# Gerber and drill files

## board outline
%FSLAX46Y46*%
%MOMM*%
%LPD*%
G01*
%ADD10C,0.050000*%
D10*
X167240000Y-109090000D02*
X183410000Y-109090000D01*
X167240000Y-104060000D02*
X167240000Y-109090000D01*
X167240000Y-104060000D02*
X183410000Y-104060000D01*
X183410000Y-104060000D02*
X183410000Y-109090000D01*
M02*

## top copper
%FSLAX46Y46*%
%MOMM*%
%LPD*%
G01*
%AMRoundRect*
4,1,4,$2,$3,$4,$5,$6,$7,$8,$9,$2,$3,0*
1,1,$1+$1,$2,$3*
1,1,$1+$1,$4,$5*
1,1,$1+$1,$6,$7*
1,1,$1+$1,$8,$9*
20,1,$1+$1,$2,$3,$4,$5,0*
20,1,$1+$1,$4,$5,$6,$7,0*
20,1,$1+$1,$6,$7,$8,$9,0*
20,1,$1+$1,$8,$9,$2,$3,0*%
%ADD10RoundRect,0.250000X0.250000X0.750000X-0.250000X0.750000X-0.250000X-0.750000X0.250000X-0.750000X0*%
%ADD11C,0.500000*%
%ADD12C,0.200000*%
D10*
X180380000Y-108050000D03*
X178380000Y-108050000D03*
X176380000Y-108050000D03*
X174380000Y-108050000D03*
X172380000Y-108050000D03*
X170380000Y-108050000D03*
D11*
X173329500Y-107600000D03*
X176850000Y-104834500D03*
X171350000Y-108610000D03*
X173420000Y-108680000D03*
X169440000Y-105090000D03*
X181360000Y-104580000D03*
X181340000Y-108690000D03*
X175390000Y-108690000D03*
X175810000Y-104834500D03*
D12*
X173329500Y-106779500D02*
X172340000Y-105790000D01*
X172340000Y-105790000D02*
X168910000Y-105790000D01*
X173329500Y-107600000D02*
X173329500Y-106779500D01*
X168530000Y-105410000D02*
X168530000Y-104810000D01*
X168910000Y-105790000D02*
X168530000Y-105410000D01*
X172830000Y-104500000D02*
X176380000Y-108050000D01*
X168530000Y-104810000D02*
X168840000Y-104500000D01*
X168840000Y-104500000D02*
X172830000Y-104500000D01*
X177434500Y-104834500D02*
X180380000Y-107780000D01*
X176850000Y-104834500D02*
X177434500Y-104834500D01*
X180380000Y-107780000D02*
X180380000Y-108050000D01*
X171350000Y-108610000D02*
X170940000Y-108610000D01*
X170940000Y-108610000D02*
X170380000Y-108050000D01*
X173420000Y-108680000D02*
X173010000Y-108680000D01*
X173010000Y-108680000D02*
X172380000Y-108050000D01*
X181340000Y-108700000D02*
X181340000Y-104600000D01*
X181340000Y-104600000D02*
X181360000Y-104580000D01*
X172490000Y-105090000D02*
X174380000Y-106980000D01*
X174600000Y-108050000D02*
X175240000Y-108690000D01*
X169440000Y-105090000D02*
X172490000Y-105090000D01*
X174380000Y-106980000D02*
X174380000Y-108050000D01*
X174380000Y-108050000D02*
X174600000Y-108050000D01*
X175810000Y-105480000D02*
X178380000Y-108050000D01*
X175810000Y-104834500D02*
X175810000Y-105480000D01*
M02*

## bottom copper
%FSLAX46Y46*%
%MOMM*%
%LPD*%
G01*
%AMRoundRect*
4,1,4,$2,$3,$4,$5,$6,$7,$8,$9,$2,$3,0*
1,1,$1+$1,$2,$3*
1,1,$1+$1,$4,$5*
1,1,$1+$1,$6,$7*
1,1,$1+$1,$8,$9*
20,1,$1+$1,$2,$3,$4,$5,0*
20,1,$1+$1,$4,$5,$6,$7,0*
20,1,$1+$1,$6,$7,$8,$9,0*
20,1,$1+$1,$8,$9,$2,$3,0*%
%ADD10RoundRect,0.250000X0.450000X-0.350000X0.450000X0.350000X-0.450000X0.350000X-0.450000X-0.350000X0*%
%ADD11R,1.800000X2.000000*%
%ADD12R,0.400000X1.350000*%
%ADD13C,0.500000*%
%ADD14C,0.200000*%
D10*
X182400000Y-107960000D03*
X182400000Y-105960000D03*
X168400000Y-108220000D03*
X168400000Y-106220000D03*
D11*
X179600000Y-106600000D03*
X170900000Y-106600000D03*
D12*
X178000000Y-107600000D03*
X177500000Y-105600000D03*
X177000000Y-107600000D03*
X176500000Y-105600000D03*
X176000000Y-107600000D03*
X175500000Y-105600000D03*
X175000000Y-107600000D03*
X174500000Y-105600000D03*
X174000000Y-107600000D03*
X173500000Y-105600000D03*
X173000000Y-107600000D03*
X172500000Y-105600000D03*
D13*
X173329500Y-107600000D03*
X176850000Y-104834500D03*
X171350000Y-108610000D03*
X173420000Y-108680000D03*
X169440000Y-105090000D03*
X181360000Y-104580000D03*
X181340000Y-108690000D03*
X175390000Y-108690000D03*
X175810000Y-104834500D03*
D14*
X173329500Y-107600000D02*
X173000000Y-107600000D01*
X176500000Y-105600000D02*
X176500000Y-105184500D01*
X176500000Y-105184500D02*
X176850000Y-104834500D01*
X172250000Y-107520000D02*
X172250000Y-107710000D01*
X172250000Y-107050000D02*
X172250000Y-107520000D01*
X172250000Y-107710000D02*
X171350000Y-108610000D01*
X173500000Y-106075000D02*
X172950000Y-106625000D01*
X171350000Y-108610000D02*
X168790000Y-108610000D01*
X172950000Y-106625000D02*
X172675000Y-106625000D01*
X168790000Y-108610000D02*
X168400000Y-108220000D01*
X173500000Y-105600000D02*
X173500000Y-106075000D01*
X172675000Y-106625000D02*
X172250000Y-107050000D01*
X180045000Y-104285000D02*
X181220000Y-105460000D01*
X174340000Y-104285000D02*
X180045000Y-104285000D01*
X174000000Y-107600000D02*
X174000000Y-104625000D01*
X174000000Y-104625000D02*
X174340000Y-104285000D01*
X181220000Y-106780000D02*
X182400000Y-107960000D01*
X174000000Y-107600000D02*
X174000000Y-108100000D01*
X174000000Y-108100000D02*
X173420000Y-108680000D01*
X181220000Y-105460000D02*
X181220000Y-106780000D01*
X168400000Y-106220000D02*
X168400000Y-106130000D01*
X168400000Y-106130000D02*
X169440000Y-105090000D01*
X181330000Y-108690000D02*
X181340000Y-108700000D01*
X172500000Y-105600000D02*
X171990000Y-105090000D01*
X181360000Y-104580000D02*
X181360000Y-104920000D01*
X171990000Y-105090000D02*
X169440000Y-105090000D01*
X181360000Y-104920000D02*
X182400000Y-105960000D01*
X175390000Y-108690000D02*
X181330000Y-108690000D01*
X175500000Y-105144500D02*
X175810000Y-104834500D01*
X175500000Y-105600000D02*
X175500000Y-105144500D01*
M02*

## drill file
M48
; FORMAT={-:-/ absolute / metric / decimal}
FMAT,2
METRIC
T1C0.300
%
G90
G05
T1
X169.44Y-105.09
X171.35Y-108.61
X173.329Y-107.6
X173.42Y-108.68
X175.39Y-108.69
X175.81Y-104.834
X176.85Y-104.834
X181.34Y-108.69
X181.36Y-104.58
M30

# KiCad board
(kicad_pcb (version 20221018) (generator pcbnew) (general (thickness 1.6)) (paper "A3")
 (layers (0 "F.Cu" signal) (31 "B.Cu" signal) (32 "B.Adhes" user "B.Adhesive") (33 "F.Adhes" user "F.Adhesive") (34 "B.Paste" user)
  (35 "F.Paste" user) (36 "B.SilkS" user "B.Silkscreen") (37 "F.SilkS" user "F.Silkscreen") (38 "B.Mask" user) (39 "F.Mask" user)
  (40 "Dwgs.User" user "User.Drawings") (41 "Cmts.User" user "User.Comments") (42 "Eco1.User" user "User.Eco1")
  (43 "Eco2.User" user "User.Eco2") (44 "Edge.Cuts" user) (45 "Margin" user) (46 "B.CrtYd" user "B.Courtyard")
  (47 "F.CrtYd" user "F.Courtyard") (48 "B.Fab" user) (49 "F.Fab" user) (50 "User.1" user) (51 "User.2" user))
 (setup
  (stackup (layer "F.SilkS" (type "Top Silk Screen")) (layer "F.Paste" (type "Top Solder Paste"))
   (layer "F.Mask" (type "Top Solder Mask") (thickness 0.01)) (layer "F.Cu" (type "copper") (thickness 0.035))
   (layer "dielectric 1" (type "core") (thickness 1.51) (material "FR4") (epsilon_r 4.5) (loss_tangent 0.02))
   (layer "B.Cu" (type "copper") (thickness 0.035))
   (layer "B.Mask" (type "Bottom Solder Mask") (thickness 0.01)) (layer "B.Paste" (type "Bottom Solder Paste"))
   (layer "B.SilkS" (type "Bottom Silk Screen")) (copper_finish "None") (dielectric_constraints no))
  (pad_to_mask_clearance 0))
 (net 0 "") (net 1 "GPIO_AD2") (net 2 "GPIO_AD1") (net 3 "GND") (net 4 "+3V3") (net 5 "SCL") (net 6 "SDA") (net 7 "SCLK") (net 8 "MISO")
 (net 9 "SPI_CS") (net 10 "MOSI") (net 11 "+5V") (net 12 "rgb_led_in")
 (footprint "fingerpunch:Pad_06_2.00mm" (layer "F.Cu") (at 175.38 108.05 180)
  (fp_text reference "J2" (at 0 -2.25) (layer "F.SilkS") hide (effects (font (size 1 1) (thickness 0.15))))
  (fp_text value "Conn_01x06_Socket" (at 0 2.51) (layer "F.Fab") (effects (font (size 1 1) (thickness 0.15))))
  (pad "1" smd roundrect (at -5 0 180) (size 1 2) (layers "F.Cu" "F.Paste" "F.Mask") (roundrect_rratio 0.25) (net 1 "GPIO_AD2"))
  (pad "2" smd roundrect (at -3 0 180) (size 1 2) (layers "F.Cu" "F.Paste" "F.Mask") (roundrect_rratio 0.25) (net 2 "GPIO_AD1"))
  (pad "3" smd roundrect (at -1 0 180) (size 1 2) (layers "F.Cu" "F.Paste" "F.Mask") (roundrect_rratio 0.25) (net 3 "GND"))
  (pad "4" smd roundrect (at 1 0 180) (size 1 2) (layers "F.Cu" "F.Paste" "F.Mask") (roundrect_rratio 0.25) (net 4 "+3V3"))
  (pad "5" smd roundrect (at 3 0 180) (size 1 2) (layers "F.Cu" "F.Paste" "F.Mask") (roundrect_rratio 0.25) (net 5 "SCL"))
  (pad "6" smd roundrect (at 5 0 180) (size 1 2) (layers "F.Cu" "F.Paste" "F.Mask") (roundrect_rratio 0.25) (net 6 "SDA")))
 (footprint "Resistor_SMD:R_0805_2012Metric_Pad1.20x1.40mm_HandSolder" (layer "B.Cu") (at 182.4 106.96 90)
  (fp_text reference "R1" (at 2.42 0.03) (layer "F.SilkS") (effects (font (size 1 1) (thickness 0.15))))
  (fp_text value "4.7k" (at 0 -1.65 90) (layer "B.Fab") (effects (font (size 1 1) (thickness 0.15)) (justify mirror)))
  (pad "1" smd roundrect (at -1 0 90) (size 1.2 1.4) (layers "B.Cu" "B.Paste" "B.Mask") (roundrect_rratio 0.2083333333) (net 5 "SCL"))
  (pad "2" smd roundrect (at 1 0 90) (size 1.2 1.4) (layers "B.Cu" "B.Paste" "B.Mask") (roundrect_rratio 0.2083333333) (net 4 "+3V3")))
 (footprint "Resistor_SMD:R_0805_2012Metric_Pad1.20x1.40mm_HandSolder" (layer "B.Cu") (at 168.4 107.22 90)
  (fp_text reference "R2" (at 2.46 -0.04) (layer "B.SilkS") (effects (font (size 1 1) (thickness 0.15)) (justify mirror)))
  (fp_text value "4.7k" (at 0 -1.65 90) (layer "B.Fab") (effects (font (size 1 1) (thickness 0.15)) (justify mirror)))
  (pad "1" smd roundrect (at -1 0 90) (size 1.2 1.4) (layers "B.Cu" "B.Paste" "B.Mask") (roundrect_rratio 0.2083333333) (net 6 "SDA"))
  (pad "2" smd roundrect (at 1 0 90) (size 1.2 1.4) (layers "B.Cu" "B.Paste" "B.Mask") (roundrect_rratio 0.2083333333) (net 4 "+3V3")))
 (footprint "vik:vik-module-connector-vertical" (layer "B.Cu") (at 175.25 106.6 180)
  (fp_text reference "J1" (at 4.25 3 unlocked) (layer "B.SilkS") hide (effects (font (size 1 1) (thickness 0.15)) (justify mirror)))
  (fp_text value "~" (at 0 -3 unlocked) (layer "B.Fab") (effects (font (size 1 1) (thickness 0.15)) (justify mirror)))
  (pad "" smd rect (at -4.35 0 180) (size 1.8 2) (layers "B.Cu" "B.Paste" "B.Mask") (thermal_bridge_angle 45))
  (pad "" smd rect (at 4.35 0 180) (size 1.8 2) (layers "B.Cu" "B.Paste" "B.Mask") (thermal_bridge_angle 45))
  (pad "1" smd rect (at -2.75 -1 180) (size 0.4 1.35) (layers "B.Cu" "B.Paste" "B.Mask") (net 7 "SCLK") (thermal_bridge_angle 45))
  (pad "2" smd rect (at -2.25 1 180) (size 0.4 1.35) (layers "B.Cu" "B.Paste" "B.Mask") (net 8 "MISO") (thermal_bridge_angle 45))
  (pad "3" smd rect (at -1.75 -1 180) (size 0.4 1.35) (layers "B.Cu" "B.Paste" "B.Mask") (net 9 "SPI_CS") (thermal_bridge_angle 45))
  (pad "4" smd rect (at -1.25 1 180) (size 0.4 1.35) (layers "B.Cu" "B.Paste" "B.Mask") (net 1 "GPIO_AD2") (thermal_bridge_angle 45))
  (pad "5" smd rect (at -0.75 -1 180) (size 0.4 1.35) (layers "B.Cu" "B.Paste" "B.Mask") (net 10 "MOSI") (thermal_bridge_angle 45))
  (pad "6" smd rect (at -0.25 1 180) (size 0.4 1.35) (layers "B.Cu" "B.Paste" "B.Mask") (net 2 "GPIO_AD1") (thermal_bridge_angle 45))
  (pad "7" smd rect (at 0.25 -1 180) (size 0.4 1.35) (layers "B.Cu" "B.Paste" "B.Mask") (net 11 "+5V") (thermal_bridge_angle 45))
  (pad "8" smd rect (at 0.75 1 180) (size 0.4 1.35) (layers "B.Cu" "B.Paste" "B.Mask") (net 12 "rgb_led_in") (thermal_bridge_angle 45))
  (pad "9" smd rect (at 1.25 -1 180) (size 0.4 1.35) (layers "B.Cu" "B.Paste" "B.Mask") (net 5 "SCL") (thermal_bridge_angle 45))
  (pad "10" smd rect (at 1.75 1 180) (size 0.4 1.35) (layers "B.Cu" "B.Paste" "B.Mask") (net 6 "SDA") (thermal_bridge_angle 45))
  (pad "11" smd rect (at 2.25 -1 180) (size 0.4 1.35) (layers "B.Cu" "B.Paste" "B.Mask") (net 3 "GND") (thermal_bridge_angle 45))
  (pad "12" smd rect (at 2.75 1 180) (size 0.4 1.35) (layers "B.Cu" "B.Paste" "B.Mask") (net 4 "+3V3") (thermal_bridge_angle 45)))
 (gr_line (start 167.24 109.09) (end 183.41 109.09) (stroke (width 0.05) (type default)) (layer "Edge.Cuts"))
 (gr_line (start 167.24 104.06) (end 167.24 109.09) (stroke (width 0.05) (type default)) (layer "Edge.Cuts"))
 (gr_line (start 167.24 104.06) (end 183.41 104.06) (stroke (width 0.05) (type default)) (layer "Edge.Cuts"))
 (gr_line (start 183.41 104.06) (end 183.41 109.09) (stroke (width 0.05) (type default)) (layer "Edge.Cuts"))
 (segment (start 173.3295 106.7795) (end 172.34 105.79) (width 0.2) (layer "F.Cu") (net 3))
 (segment (start 172.34 105.79) (end 168.91 105.79) (width 0.2) (layer "F.Cu") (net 3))
 (segment (start 173.3295 107.6) (end 173.3295 106.7795) (width 0.2) (layer "F.Cu") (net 3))
 (segment (start 168.53 105.41) (end 168.53 104.81) (width 0.2) (layer "F.Cu") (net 3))
 (segment (start 168.91 105.79) (end 168.53 105.41) (width 0.2) (layer "F.Cu") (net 3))
 (segment (start 172.83 104.5) (end 176.38 108.05) (width 0.2) (layer "F.Cu") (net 3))
 (segment (start 168.53 104.81) (end 168.84 104.5) (width 0.2) (layer "F.Cu") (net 3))
 (segment (start 168.84 104.5) (end 172.83 104.5) (width 0.2) (layer "F.Cu") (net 3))
 (via (at 173.3295 107.6) (size 0.5) (drill 0.3) (layers "F.Cu" "B.Cu") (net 3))
 (segment (start 173.3295 107.6) (end 173 107.6) (width 0.2) (layer "B.Cu") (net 3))
 (segment (start 177.4345 104.8345) (end 180.38 107.78) (width 0.2) (layer "F.Cu") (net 1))
 (segment (start 176.85 104.8345) (end 177.4345 104.8345) (width 0.2) (layer "F.Cu") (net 1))
 (segment (start 180.38 107.78) (end 180.38 108.05) (width 0.2) (layer "F.Cu") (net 1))
 (via (at 176.85 104.8345) (size 0.5) (drill 0.3) (layers "F.Cu" "B.Cu") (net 1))
 (segment (start 176.5 105.6) (end 176.5 105.1845) (width 0.2) (layer "B.Cu") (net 1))
 (segment (start 176.5 105.1845) (end 176.85 104.8345) (width 0.2) (layer "B.Cu") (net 1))
 (segment (start 171.35 108.61) (end 170.94 108.61) (width 0.2) (layer "F.Cu") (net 6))
 (segment (start 170.94 108.61) (end 170.38 108.05) (width 0.2) (layer "F.Cu") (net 6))
 (via (at 171.35 108.61) (size 0.5) (drill 0.3) (layers "F.Cu" "B.Cu") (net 6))
 (segment (start 172.25 107.52) (end 172.25 107.71) (width 0.2) (layer "B.Cu") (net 6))
 (segment (start 172.25 107.05) (end 172.25 107.52) (width 0.2) (layer "B.Cu") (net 6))
 (segment (start 172.25 107.71) (end 171.35 108.61) (width 0.2) (layer "B.Cu") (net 6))
 (segment (start 173.5 106.075) (end 172.95 106.625) (width 0.2) (layer "B.Cu") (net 6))
 (segment (start 171.35 108.61) (end 168.79 108.61) (width 0.2) (layer "B.Cu") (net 6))
 (segment (start 172.95 106.625) (end 172.675 106.625) (width 0.2) (layer "B.Cu") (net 6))
 (segment (start 168.79 108.61) (end 168.4 108.22) (width 0.2) (layer "B.Cu") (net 6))
 (segment (start 173.5 105.6) (end 173.5 106.075) (width 0.2) (layer "B.Cu") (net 6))
 (segment (start 172.675 106.625) (end 172.25 107.05) (width 0.2) (layer "B.Cu") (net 6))
 (segment (start 173.42 108.68) (end 173.01 108.68) (width 0.2) (layer "F.Cu") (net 5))
 (segment (start 173.01 108.68) (end 172.38 108.05) (width 0.2) (layer "F.Cu") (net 5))
 (via (at 173.42 108.68) (size 0.5) (drill 0.3) (layers "F.Cu" "B.Cu") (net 5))
 (segment (start 180.045 104.285) (end 181.22 105.46) (width 0.2) (layer "B.Cu") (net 5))
 (segment (start 174.34 104.285) (end 180.045 104.285) (width 0.2) (layer "B.Cu") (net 5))
 (segment (start 174 107.6) (end 174 104.625) (width 0.2) (layer "B.Cu") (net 5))
 (segment (start 174 104.625) (end 174.34 104.285) (width 0.2) (layer "B.Cu") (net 5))
 (segment (start 181.22 106.78) (end 182.4 107.96) (width 0.2) (layer "B.Cu") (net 5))
 (segment (start 174 107.6) (end 174 108.1) (width 0.2) (layer "B.Cu") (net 5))
 (segment (start 174 108.1) (end 173.42 108.68) (width 0.2) (layer "B.Cu") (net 5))
 (segment (start 181.22 105.46) (end 181.22 106.78) (width 0.2) (layer "B.Cu") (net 5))
 (segment (start 181.34 108.7) (end 181.34 104.6) (width 0.2) (layer "F.Cu") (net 4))
 (segment (start 181.34 104.6) (end 181.36 104.58) (width 0.2) (layer "F.Cu") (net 4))
 (segment (start 172.49 105.09) (end 174.38 106.98) (width 0.2) (layer "F.Cu") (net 4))
 (segment (start 174.6 108.05) (end 175.24 108.69) (width 0.2) (layer "F.Cu") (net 4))
 (segment (start 169.44 105.09) (end 172.49 105.09) (width 0.2) (layer "F.Cu") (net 4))
 (segment (start 174.38 106.98) (end 174.38 108.05) (width 0.2) (layer "F.Cu") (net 4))
 (segment (start 174.38 108.05) (end 174.6 108.05) (width 0.2) (layer "F.Cu") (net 4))
 (via (at 169.44 105.09) (size 0.5) (drill 0.3) (layers "F.Cu" "B.Cu") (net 4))
 (via (at 181.36 104.58) (size 0.5) (drill 0.3) (layers "F.Cu" "B.Cu") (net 4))
 (via (at 181.34 108.69) (size 0.5) (drill 0.3) (layers "F.Cu" "B.Cu") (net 4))
 (via (at 175.39 108.69) (size 0.5) (drill 0.3) (layers "F.Cu" "B.Cu") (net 4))
 (segment (start 168.4 106.22) (end 168.4 106.13) (width 0.2) (layer "B.Cu") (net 4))
 (segment (start 168.4 106.13) (end 169.44 105.09) (width 0.2) (layer "B.Cu") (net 4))
 (segment (start 181.33 108.69) (end 181.34 108.7) (width 0.2) (layer "B.Cu") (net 4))
 (segment (start 172.5 105.6) (end 171.99 105.09) (width 0.2) (layer "B.Cu") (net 4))
 (segment (start 181.36 104.58) (end 181.36 104.92) (width 0.2) (layer "B.Cu") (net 4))
 (segment (start 171.99 105.09) (end 169.44 105.09) (width 0.2) (layer "B.Cu") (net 4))
 (segment (start 181.36 104.92) (end 182.4 105.96) (width 0.2) (layer "B.Cu") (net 4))
 (segment (start 175.39 108.69) (end 181.33 108.69) (width 0.2) (layer "B.Cu") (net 4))
 (segment (start 175.81 105.48) (end 178.38 108.05) (width 0.2) (layer "F.Cu") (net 2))
 (segment (start 175.81 104.8345) (end 175.81 105.48) (width 0.2) (layer "F.Cu") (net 2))
 (via (at 175.81 104.8345) (size 0.5) (drill 0.3) (layers "F.Cu" "B.Cu") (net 2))
 (segment (start 175.5 105.1445) (end 175.81 104.8345) (width 0.2) (layer "B.Cu") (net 2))
 (segment (start 175.5 105.6) (end 175.5 105.1445) (width 0.2) (layer "B.Cu") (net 2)))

